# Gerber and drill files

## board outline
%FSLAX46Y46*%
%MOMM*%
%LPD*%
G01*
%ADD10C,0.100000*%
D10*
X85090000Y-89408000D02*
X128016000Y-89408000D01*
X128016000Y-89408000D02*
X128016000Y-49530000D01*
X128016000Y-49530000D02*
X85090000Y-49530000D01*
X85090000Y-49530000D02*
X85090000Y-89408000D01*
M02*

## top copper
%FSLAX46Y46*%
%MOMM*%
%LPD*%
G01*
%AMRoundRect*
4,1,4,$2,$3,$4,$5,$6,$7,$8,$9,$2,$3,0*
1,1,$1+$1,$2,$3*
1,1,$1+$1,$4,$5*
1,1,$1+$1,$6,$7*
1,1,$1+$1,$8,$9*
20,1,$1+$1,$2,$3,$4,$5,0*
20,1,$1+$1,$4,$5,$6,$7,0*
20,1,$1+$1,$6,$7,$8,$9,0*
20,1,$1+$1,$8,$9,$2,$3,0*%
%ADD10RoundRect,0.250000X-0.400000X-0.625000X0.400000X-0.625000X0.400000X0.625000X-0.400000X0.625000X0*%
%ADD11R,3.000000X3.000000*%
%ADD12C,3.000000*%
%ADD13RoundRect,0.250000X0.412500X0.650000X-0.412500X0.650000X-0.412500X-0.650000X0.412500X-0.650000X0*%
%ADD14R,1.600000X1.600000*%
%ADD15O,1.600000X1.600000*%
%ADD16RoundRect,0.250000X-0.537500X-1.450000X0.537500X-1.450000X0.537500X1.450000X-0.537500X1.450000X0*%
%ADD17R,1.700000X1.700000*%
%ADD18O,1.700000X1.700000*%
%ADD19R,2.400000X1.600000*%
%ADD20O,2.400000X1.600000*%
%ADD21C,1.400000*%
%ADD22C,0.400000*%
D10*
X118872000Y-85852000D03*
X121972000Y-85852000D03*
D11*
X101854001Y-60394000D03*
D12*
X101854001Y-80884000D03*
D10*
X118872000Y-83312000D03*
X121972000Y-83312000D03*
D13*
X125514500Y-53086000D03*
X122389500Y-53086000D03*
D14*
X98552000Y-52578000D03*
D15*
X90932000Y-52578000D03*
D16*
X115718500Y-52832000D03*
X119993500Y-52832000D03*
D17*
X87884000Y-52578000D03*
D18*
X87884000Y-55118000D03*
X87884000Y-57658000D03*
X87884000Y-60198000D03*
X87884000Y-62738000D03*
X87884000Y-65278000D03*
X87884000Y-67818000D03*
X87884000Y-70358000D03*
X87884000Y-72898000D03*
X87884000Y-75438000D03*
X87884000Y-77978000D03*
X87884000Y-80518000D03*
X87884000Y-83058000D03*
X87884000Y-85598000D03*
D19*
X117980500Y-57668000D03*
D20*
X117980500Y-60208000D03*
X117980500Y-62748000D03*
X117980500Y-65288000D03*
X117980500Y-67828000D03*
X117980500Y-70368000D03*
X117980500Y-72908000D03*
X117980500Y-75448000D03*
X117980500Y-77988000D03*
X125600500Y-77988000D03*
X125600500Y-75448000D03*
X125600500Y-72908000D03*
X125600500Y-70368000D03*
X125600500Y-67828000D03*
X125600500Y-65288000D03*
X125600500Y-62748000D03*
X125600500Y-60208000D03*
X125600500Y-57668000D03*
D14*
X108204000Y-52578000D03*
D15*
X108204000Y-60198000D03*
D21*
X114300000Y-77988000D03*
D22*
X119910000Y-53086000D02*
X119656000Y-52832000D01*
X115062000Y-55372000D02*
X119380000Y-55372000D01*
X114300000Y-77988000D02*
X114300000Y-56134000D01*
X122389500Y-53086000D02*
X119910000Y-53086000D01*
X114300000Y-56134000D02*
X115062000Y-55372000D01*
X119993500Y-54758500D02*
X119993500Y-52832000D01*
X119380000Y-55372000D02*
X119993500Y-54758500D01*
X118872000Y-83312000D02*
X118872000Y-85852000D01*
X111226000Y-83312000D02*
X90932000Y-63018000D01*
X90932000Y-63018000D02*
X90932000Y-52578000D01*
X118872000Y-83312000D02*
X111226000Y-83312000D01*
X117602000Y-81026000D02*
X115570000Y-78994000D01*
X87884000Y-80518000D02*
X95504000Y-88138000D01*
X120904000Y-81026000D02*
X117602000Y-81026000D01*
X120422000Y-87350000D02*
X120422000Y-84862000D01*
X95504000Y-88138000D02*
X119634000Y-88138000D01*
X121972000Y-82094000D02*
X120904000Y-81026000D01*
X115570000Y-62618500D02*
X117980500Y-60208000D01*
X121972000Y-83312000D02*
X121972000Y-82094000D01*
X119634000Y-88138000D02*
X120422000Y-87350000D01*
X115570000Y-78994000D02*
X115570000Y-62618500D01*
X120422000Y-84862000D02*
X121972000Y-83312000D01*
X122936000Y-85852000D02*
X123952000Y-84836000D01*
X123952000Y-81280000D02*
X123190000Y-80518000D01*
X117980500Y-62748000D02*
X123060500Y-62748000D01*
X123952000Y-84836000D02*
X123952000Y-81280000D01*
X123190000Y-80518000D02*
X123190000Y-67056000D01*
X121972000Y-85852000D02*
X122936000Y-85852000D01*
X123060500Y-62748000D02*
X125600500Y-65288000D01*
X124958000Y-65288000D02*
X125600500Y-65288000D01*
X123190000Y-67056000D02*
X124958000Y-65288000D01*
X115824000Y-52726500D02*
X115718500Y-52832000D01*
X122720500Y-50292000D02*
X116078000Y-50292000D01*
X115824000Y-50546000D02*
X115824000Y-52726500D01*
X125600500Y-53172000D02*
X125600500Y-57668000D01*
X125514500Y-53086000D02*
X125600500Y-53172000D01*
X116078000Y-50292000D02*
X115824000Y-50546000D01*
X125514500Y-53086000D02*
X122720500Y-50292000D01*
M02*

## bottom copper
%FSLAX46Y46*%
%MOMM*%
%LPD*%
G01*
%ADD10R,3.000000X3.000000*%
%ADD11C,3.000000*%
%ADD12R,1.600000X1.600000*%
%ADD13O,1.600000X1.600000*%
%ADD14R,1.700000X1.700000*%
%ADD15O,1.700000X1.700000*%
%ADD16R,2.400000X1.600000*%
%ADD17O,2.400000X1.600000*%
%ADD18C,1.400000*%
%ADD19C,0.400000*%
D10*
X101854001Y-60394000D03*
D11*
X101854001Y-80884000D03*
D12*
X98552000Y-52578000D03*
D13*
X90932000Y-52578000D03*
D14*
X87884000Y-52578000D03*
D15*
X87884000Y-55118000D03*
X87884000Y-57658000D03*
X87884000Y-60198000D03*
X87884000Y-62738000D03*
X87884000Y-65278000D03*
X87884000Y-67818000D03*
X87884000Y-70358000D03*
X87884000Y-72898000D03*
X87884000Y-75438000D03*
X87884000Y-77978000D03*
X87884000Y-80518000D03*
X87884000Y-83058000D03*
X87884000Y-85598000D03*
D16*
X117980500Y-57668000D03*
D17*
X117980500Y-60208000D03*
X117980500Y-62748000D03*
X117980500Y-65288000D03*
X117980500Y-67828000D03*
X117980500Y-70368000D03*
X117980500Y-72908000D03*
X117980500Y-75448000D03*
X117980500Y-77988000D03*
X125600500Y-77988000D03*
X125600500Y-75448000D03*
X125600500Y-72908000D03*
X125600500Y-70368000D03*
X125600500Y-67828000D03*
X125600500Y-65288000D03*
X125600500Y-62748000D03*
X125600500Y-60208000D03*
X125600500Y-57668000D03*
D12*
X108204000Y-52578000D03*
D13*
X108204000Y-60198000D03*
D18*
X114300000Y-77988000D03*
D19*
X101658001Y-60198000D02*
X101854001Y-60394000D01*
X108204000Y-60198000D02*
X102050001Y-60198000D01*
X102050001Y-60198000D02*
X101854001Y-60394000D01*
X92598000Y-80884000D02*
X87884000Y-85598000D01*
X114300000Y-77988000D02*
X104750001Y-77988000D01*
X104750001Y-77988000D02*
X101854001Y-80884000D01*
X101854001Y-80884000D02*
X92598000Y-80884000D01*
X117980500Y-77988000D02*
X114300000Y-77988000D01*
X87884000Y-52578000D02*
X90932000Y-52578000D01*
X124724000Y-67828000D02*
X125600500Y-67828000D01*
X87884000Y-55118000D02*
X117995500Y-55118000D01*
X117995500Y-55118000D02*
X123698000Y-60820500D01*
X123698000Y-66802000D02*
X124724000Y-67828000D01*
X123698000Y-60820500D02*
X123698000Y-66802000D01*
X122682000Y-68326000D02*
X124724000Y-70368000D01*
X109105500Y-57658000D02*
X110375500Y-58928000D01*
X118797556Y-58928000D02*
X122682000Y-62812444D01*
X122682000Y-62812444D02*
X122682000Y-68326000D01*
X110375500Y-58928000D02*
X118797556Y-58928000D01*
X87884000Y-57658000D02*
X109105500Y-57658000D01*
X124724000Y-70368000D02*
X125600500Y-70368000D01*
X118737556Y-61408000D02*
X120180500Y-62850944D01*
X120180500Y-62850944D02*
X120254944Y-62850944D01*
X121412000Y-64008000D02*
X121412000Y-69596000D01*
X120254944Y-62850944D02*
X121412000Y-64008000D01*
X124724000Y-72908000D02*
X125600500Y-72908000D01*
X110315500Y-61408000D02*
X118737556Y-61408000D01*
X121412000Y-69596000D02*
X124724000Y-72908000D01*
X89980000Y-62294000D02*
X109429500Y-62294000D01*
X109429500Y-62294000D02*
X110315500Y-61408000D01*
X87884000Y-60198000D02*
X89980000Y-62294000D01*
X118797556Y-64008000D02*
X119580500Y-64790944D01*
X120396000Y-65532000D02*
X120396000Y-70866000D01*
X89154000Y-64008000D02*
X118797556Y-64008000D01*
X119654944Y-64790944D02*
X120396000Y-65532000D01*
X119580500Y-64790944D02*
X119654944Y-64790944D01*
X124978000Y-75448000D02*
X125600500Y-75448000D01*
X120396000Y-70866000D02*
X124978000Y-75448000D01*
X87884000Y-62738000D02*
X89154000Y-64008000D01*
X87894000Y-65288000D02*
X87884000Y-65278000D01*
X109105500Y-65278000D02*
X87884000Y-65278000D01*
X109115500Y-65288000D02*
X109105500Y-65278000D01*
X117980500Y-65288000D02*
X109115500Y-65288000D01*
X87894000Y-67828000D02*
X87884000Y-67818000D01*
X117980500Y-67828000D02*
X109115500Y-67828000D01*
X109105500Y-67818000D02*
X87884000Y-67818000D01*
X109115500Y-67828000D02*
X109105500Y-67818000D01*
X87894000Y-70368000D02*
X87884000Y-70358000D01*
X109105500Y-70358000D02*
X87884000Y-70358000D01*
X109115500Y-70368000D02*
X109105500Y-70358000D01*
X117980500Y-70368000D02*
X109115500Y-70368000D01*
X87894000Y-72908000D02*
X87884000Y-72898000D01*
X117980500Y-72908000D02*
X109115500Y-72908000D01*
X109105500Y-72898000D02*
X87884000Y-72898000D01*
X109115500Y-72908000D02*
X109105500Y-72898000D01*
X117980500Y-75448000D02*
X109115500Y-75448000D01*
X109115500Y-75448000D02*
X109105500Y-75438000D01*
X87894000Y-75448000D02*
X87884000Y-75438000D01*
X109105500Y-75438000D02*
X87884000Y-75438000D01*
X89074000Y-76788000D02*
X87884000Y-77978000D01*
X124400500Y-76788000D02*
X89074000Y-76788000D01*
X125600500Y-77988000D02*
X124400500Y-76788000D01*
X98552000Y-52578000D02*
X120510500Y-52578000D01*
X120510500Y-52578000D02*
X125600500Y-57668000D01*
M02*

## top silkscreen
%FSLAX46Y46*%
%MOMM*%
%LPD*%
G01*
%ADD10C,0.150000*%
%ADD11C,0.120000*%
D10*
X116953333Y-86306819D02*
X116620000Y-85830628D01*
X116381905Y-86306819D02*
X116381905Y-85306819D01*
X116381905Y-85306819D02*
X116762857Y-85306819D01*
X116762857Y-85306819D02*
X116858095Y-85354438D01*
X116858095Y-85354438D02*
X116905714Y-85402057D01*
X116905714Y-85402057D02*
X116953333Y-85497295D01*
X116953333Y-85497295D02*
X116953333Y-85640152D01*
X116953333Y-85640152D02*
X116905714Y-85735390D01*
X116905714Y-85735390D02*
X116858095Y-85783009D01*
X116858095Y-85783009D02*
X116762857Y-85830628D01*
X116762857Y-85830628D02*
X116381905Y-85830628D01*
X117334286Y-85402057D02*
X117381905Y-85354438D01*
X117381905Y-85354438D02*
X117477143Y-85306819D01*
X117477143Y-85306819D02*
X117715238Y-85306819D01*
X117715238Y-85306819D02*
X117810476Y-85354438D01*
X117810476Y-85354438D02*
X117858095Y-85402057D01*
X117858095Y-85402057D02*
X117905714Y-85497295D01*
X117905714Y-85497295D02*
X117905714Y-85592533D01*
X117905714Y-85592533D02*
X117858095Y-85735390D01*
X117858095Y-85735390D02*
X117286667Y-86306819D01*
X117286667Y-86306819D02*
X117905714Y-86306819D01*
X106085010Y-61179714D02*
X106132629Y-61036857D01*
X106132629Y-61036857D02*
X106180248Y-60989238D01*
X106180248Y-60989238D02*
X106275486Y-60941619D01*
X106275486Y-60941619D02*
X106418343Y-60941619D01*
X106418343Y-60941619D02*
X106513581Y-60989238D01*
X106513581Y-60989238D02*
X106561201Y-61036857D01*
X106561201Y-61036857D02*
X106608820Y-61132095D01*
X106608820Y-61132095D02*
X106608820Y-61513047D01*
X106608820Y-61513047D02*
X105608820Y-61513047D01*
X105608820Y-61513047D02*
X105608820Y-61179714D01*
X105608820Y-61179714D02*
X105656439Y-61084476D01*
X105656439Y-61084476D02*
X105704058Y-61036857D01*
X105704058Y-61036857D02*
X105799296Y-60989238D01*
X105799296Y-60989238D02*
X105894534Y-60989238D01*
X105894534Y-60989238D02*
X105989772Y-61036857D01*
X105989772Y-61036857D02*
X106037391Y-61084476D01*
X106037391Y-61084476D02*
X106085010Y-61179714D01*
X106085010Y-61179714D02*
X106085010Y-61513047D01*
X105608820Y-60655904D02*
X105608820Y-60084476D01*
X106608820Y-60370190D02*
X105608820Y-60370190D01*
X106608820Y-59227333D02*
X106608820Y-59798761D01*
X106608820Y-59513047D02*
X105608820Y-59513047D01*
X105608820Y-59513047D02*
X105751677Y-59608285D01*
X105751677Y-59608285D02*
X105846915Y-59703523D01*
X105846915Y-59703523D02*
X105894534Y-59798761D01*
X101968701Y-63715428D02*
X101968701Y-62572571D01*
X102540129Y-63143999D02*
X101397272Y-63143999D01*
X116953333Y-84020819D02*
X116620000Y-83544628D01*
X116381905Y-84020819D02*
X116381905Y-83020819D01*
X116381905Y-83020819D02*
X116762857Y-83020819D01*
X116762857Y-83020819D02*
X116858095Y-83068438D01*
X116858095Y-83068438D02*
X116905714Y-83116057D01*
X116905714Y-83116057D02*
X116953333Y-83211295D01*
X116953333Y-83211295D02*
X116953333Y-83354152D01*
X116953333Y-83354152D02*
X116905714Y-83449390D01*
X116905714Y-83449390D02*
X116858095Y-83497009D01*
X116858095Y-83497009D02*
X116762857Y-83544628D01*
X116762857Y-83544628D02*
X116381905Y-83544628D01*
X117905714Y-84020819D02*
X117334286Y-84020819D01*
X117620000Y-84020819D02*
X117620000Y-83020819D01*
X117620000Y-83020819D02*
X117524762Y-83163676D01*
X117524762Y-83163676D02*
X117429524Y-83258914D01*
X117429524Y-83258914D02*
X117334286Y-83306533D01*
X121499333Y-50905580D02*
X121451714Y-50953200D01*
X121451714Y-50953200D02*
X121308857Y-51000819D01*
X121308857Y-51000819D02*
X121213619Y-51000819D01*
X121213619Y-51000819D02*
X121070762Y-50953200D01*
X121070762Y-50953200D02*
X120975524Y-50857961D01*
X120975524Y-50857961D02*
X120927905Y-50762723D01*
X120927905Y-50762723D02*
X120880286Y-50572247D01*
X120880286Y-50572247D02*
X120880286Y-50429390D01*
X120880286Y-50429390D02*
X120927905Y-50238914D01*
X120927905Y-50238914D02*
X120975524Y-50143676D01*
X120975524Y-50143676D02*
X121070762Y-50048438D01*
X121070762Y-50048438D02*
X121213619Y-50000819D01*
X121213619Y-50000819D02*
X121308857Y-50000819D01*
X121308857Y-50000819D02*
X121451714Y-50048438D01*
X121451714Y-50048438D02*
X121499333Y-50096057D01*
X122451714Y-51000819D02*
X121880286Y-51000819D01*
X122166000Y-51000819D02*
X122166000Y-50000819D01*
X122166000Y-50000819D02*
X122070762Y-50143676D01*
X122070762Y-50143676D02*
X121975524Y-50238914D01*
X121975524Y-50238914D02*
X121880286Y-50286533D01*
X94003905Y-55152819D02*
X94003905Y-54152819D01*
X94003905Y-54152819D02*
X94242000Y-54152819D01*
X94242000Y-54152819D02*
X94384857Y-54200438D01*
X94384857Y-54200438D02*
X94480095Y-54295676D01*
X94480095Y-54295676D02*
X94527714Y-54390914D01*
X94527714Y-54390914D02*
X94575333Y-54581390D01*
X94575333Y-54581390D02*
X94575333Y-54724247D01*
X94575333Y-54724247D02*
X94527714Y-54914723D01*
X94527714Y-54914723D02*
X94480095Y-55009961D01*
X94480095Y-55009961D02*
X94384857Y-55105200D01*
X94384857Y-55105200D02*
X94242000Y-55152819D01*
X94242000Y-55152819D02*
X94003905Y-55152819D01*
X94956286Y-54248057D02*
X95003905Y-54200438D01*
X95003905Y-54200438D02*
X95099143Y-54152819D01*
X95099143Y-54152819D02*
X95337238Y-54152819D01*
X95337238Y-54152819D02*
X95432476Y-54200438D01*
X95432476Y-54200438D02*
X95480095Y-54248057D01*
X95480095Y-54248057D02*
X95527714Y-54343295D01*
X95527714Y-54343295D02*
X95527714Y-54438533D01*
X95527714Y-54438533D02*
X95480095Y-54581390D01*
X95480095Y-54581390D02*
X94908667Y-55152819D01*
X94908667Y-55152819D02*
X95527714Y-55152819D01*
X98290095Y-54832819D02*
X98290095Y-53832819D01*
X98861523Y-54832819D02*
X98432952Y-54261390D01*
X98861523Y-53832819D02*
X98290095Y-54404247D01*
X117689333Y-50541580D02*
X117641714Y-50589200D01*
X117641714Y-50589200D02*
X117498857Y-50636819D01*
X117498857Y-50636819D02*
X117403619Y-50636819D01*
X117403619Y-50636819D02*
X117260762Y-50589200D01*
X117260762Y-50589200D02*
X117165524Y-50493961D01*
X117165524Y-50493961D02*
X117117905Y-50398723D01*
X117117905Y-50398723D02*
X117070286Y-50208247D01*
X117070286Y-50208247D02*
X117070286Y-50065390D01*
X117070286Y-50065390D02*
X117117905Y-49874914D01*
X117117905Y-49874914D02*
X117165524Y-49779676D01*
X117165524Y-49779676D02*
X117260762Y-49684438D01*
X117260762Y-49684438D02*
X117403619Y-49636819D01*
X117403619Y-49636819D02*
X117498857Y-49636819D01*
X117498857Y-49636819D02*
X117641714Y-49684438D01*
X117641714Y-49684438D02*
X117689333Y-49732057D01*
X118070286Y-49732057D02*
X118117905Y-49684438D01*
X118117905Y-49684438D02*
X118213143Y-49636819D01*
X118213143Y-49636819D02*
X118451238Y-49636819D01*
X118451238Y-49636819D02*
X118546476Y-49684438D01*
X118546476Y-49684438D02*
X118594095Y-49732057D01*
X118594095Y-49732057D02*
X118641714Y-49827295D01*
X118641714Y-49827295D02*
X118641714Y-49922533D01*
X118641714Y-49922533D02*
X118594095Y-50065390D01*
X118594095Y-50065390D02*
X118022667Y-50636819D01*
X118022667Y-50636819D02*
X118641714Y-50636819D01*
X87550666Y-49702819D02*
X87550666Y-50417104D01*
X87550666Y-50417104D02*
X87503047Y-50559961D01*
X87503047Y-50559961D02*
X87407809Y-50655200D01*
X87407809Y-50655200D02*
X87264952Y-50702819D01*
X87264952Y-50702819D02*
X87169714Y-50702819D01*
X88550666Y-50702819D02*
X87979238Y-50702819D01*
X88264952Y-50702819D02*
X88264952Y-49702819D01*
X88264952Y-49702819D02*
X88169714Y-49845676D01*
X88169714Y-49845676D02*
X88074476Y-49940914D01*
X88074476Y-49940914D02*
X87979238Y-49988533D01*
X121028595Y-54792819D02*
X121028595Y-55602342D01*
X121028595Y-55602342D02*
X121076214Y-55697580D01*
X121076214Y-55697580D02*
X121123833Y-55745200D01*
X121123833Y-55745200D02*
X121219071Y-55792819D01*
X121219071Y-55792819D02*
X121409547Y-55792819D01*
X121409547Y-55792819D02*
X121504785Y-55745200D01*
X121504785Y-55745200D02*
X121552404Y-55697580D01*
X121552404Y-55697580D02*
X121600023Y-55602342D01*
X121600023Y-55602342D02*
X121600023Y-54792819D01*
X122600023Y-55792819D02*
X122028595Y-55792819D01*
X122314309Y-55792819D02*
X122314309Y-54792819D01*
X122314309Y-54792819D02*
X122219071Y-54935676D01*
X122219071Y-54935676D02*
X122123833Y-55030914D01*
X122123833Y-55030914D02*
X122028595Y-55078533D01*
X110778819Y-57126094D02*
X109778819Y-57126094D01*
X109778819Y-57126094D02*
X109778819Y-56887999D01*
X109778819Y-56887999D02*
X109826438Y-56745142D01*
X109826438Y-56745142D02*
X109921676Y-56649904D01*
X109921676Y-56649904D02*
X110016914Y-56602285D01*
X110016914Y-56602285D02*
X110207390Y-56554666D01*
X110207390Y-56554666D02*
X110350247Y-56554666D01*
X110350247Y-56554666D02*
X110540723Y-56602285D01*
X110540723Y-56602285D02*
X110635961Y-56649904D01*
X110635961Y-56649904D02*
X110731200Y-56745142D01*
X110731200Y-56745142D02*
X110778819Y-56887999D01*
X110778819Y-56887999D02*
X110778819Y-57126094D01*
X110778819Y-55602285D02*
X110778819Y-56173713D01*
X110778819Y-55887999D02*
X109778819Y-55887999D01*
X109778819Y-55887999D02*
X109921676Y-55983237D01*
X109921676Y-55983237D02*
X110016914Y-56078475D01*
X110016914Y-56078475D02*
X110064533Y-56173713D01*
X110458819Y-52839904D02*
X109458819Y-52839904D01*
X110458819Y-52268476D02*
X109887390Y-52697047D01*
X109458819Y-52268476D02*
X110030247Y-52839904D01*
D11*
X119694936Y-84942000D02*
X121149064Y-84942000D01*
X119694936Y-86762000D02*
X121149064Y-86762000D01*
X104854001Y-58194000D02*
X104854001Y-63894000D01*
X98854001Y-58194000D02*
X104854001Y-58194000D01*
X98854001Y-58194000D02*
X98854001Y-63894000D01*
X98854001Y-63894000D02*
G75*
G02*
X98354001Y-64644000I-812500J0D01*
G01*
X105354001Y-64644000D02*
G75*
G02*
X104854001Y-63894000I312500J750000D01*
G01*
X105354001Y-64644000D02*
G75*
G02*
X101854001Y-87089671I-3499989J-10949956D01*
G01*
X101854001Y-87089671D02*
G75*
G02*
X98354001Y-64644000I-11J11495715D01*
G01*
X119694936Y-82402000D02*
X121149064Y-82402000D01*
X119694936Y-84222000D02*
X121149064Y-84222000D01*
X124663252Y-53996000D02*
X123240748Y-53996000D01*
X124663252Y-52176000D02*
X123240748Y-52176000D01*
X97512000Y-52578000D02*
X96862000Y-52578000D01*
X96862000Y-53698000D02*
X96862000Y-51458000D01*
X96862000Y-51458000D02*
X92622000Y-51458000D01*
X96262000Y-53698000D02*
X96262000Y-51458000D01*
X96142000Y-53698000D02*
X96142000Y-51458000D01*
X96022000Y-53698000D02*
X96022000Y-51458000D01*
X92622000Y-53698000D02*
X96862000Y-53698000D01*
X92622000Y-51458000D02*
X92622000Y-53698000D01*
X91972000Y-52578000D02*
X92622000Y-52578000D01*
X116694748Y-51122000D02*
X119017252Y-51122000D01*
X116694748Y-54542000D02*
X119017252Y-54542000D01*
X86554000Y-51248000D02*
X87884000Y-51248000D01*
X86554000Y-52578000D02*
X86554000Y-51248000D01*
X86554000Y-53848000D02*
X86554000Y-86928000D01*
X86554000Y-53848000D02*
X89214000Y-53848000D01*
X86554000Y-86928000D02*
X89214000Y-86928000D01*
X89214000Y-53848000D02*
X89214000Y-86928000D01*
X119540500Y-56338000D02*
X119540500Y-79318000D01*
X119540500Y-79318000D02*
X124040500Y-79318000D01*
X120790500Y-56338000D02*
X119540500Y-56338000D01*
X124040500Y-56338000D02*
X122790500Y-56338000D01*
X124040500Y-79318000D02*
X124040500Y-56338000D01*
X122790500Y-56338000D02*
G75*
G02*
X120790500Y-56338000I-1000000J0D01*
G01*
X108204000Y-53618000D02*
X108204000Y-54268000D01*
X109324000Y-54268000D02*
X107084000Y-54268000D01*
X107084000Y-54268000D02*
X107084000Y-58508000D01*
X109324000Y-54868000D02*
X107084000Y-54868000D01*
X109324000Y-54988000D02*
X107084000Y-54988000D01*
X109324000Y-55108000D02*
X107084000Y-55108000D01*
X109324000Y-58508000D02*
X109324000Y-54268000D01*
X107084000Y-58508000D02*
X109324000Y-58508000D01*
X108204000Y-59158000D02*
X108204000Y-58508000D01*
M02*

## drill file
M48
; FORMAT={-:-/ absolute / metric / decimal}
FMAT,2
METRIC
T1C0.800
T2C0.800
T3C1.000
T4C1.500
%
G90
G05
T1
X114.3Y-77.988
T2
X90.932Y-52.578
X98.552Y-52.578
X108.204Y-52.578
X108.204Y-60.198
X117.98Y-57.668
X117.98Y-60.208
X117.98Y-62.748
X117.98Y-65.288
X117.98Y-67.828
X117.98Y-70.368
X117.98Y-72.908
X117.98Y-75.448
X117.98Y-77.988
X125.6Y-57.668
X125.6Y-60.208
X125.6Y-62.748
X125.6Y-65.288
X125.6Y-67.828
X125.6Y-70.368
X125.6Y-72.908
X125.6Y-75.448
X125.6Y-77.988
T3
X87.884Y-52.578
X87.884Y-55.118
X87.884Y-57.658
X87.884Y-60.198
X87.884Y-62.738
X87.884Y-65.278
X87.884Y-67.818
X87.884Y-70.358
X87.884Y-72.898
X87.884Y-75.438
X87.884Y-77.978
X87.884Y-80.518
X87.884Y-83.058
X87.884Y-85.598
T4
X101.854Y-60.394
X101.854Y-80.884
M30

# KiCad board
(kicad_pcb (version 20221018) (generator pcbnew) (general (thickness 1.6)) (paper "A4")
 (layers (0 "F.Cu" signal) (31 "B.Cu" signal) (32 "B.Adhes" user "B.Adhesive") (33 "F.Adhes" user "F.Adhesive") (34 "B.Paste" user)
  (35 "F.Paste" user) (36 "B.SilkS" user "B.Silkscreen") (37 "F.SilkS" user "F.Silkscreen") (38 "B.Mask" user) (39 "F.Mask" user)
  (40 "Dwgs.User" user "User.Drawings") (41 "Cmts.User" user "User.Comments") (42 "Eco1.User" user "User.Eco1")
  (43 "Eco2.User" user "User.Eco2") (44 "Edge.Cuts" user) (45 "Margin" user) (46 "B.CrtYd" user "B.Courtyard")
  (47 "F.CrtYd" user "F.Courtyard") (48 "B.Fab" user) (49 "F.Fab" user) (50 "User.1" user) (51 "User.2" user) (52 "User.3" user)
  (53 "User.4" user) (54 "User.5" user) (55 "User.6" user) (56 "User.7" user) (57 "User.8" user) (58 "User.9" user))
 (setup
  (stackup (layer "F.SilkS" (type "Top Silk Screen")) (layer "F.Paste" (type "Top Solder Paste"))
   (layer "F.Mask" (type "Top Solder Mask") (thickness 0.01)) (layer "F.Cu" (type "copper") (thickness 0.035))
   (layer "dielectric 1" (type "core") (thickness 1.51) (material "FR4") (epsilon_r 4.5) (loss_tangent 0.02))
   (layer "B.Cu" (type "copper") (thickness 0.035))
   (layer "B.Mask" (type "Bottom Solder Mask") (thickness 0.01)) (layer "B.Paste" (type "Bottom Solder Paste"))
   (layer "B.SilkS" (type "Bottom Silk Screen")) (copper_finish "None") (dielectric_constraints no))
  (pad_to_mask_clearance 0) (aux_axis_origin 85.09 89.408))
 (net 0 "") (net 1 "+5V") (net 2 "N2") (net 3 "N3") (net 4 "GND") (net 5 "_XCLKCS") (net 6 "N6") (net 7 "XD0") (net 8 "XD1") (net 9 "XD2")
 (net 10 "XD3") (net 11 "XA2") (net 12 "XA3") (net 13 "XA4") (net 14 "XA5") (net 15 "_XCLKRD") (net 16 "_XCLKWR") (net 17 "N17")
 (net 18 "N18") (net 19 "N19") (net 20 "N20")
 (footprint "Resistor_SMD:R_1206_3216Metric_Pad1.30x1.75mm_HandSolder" (layer "F.Cu") (at 120.422 85.852)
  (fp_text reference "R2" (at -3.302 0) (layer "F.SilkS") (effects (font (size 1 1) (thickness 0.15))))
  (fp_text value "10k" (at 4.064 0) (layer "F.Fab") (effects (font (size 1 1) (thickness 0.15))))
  (fp_line (start -0.727064 -0.91) (end 0.727064 -0.91) (stroke (width 0.12) (type solid)) (layer "F.SilkS"))
  (fp_line (start -0.727064 0.91) (end 0.727064 0.91) (stroke (width 0.12) (type solid)) (layer "F.SilkS"))
  (pad "1" smd roundrect (at -1.55 0) (size 1.3 1.75) (layers "F.Cu" "F.Paste" "F.Mask") (roundrect_rratio 0.1923076923) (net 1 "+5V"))
  (pad "2" smd roundrect (at 1.55 0) (size 1.3 1.75) (layers "F.Cu" "F.Paste" "F.Mask") (roundrect_rratio 0.1923076923) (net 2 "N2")))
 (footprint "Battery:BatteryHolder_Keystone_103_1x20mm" (layer "F.Cu") (at 101.854001 60.394 -90)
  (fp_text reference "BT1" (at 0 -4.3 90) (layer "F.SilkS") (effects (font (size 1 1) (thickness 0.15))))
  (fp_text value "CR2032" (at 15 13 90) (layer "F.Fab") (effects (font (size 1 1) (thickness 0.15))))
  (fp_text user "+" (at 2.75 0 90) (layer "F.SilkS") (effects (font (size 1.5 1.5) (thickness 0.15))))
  (fp_line (start -2.2 -3) (end 3.5 -3) (stroke (width 0.12) (type solid)) (layer "F.SilkS"))
  (fp_line (start -2.2 3) (end -2.2 -3) (stroke (width 0.12) (type solid)) (layer "F.SilkS"))
  (fp_line (start -2.2 3) (end 3.5 3) (stroke (width 0.12) (type solid)) (layer "F.SilkS"))
  (fp_arc (start 3.5 3) (mid 3.950694 3.136459) (end 4.25 3.5) (stroke (width 0.12) (type solid)) (layer "F.SilkS"))
  (fp_arc (start 4.25 -3.5) (mid 3.950694 -3.136459) (end 3.5 -3) (stroke (width 0.12) (type solid)) (layer "F.SilkS"))
  (fp_arc (start 4.25 -3.5) (mid 16.971103 -11.358466) (end 26.695671 0) (stroke (width 0.12) (type solid)) (layer "F.SilkS"))
  (fp_arc (start 26.695671 0) (mid 16.971103 11.358466) (end 4.25 3.5) (stroke (width 0.12) (type solid)) (layer "F.SilkS"))
  (pad "1" thru_hole rect (at 0 0 270) (size 3 3) (drill 1.5) (layers "*.Cu" "*.Mask") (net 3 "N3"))
  (pad "2" thru_hole circle (at 20.49 0 270) (size 3 3) (drill 1.5) (layers "*.Cu" "*.Mask") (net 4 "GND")))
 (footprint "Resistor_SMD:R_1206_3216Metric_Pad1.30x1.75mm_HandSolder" (layer "F.Cu") (at 120.422 83.312)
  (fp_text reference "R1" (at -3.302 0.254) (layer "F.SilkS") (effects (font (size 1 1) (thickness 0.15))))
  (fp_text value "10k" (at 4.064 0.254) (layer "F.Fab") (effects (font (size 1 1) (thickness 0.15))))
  (fp_line (start -0.727064 -0.91) (end 0.727064 -0.91) (stroke (width 0.12) (type solid)) (layer "F.SilkS"))
  (fp_line (start -0.727064 0.91) (end 0.727064 0.91) (stroke (width 0.12) (type solid)) (layer "F.SilkS"))
  (pad "1" smd roundrect (at -1.55 0) (size 1.3 1.75) (layers "F.Cu" "F.Paste" "F.Mask") (roundrect_rratio 0.1923076923) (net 1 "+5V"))
  (pad "2" smd roundrect (at 1.55 0) (size 1.3 1.75) (layers "F.Cu" "F.Paste" "F.Mask") (roundrect_rratio 0.1923076923) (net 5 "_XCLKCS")))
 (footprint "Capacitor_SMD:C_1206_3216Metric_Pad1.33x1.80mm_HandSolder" (layer "F.Cu") (at 123.952 53.086 180)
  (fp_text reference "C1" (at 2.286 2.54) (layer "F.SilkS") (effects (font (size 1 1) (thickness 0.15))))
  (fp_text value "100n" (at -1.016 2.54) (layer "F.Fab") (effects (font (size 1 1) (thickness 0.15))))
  (fp_line (start -0.711252 -0.91) (end 0.711252 -0.91) (stroke (width 0.12) (type solid)) (layer "F.SilkS"))
  (fp_line (start -0.711252 0.91) (end 0.711252 0.91) (stroke (width 0.12) (type solid)) (layer "F.SilkS"))
  (pad "1" smd roundrect (at -1.5625 0 180) (size 1.325 1.8) (layers "F.Cu" "F.Paste" "F.Mask") (roundrect_rratio 0.1886792453) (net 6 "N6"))
  (pad "2" smd roundrect (at 1.5625 0 180) (size 1.325 1.8) (layers "F.Cu" "F.Paste" "F.Mask") (roundrect_rratio 0.1886792453) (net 4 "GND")))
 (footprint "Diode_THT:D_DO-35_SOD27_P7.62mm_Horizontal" (layer "F.Cu") (at 98.552 52.578 180)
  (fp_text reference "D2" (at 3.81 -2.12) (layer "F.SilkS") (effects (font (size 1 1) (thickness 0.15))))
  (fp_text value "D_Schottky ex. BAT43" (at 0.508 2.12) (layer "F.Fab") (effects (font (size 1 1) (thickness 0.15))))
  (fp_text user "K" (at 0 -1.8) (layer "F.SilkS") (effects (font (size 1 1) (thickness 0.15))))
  (fp_line (start 1.04 0) (end 1.69 0) (stroke (width 0.12) (type solid)) (layer "F.SilkS"))
  (fp_line (start 1.69 -1.12) (end 1.69 1.12) (stroke (width 0.12) (type solid)) (layer "F.SilkS"))
  (fp_line (start 1.69 1.12) (end 5.93 1.12) (stroke (width 0.12) (type solid)) (layer "F.SilkS"))
  (fp_line (start 2.29 -1.12) (end 2.29 1.12) (stroke (width 0.12) (type solid)) (layer "F.SilkS"))
  (fp_line (start 2.41 -1.12) (end 2.41 1.12) (stroke (width 0.12) (type solid)) (layer "F.SilkS"))
  (fp_line (start 2.53 -1.12) (end 2.53 1.12) (stroke (width 0.12) (type solid)) (layer "F.SilkS"))
  (fp_line (start 5.93 -1.12) (end 1.69 -1.12) (stroke (width 0.12) (type solid)) (layer "F.SilkS"))
  (fp_line (start 5.93 1.12) (end 5.93 -1.12) (stroke (width 0.12) (type solid)) (layer "F.SilkS"))
  (fp_line (start 6.58 0) (end 5.93 0) (stroke (width 0.12) (type solid)) (layer "F.SilkS"))
  (pad "1" thru_hole rect (at 0 0 180) (size 1.6 1.6) (drill 0.8) (layers "*.Cu" "*.Mask") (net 6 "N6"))
  (pad "2" thru_hole oval (at 7.62 0 180) (size 1.6 1.6) (drill 0.8) (layers "*.Cu" "*.Mask") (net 1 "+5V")))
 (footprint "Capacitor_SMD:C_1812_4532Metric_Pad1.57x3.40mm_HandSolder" (layer "F.Cu") (at 117.856 52.832)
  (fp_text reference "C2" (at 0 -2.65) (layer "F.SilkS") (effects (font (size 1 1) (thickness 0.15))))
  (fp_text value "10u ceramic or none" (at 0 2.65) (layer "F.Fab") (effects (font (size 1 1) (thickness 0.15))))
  (fp_line (start -1.161252 -1.71) (end 1.161252 -1.71) (stroke (width 0.12) (type solid)) (layer "F.SilkS"))
  (fp_line (start -1.161252 1.71) (end 1.161252 1.71) (stroke (width 0.12) (type solid)) (layer "F.SilkS"))
  (pad "1" smd roundrect (at -2.1375 0) (size 1.575 3.4) (layers "F.Cu" "F.Paste" "F.Mask") (roundrect_rratio 0.15873) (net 6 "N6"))
  (pad "2" smd roundrect (at 2.1375 0) (size 1.575 3.4) (layers "F.Cu" "F.Paste" "F.Mask") (roundrect_rratio 0.15873) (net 4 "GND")))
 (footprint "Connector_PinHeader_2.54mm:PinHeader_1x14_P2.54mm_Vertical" (layer "F.Cu") (at 87.884 52.578)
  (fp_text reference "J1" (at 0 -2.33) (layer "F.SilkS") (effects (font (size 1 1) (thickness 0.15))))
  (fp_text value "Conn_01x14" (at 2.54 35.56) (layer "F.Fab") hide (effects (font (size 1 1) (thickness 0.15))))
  (fp_line (start -1.33 -1.33) (end 0 -1.33) (stroke (width 0.12) (type solid)) (layer "F.SilkS"))
  (fp_line (start -1.33 0) (end -1.33 -1.33) (stroke (width 0.12) (type solid)) (layer "F.SilkS"))
  (fp_line (start -1.33 1.27) (end -1.33 34.35) (stroke (width 0.12) (type solid)) (layer "F.SilkS"))
  (fp_line (start -1.33 1.27) (end 1.33 1.27) (stroke (width 0.12) (type solid)) (layer "F.SilkS"))
  (fp_line (start -1.33 34.35) (end 1.33 34.35) (stroke (width 0.12) (type solid)) (layer "F.SilkS"))
  (fp_line (start 1.33 1.27) (end 1.33 34.35) (stroke (width 0.12) (type solid)) (layer "F.SilkS"))
  (pad "1" thru_hole rect (at 0 0) (size 1.7 1.7) (drill 1) (layers "*.Cu" "*.Mask") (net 1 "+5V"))
  (pad "2" thru_hole oval (at 0 2.54) (size 1.7 1.7) (drill 1) (layers "*.Cu" "*.Mask") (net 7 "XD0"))
  (pad "3" thru_hole oval (at 0 5.08) (size 1.7 1.7) (drill 1) (layers "*.Cu" "*.Mask") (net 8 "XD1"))
  (pad "4" thru_hole oval (at 0 7.62) (size 1.7 1.7) (drill 1) (layers "*.Cu" "*.Mask") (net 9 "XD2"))
  (pad "5" thru_hole oval (at 0 10.16) (size 1.7 1.7) (drill 1) (layers "*.Cu" "*.Mask") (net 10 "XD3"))
  (pad "6" thru_hole oval (at 0 12.7) (size 1.7 1.7) (drill 1) (layers "*.Cu" "*.Mask") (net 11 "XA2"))
  (pad "7" thru_hole oval (at 0 15.24) (size 1.7 1.7) (drill 1) (layers "*.Cu" "*.Mask") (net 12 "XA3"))
  (pad "8" thru_hole oval (at 0 17.78) (size 1.7 1.7) (drill 1) (layers "*.Cu" "*.Mask") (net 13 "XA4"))
  (pad "9" thru_hole oval (at 0 20.32) (size 1.7 1.7) (drill 1) (layers "*.Cu" "*.Mask") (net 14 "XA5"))
  (pad "10" thru_hole oval (at 0 22.86) (size 1.7 1.7) (drill 1) (layers "*.Cu" "*.Mask") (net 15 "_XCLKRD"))
  (pad "11" thru_hole oval (at 0 25.4) (size 1.7 1.7) (drill 1) (layers "*.Cu" "*.Mask") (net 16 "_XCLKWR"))
  (pad "12" thru_hole oval (at 0 27.94) (size 1.7 1.7) (drill 1) (layers "*.Cu" "*.Mask") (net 5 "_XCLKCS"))
  (pad "13" thru_hole oval (at 0 30.48) (size 1.7 1.7) (drill 1) (layers "*.Cu" "*.Mask") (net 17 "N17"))
  (pad "14" thru_hole oval (at 0 33.02) (size 1.7 1.7) (drill 1) (layers "*.Cu" "*.Mask") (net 4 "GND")))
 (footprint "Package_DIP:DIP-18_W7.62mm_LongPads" (layer "F.Cu") (at 117.9805 57.668)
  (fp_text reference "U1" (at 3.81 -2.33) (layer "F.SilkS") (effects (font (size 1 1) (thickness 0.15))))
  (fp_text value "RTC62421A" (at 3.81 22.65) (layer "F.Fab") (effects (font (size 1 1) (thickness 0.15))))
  (fp_line (start 1.56 -1.33) (end 1.56 21.65) (stroke (width 0.12) (type solid)) (layer "F.SilkS"))
  (fp_line (start 1.56 21.65) (end 6.06 21.65) (stroke (width 0.12) (type solid)) (layer "F.SilkS"))
  (fp_line (start 2.81 -1.33) (end 1.56 -1.33) (stroke (width 0.12) (type solid)) (layer "F.SilkS"))
  (fp_line (start 6.06 -1.33) (end 4.81 -1.33) (stroke (width 0.12) (type solid)) (layer "F.SilkS"))
  (fp_line (start 6.06 21.65) (end 6.06 -1.33) (stroke (width 0.12) (type solid)) (layer "F.SilkS"))
  (fp_arc (start 4.81 -1.33) (mid 3.81 -0.33) (end 2.81 -1.33) (stroke (width 0.12) (type solid)) (layer "F.SilkS"))
  (pad "1" thru_hole rect (at 0 0) (size 2.4 1.6) (drill 0.8) (layers "*.Cu" "*.Mask") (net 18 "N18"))
  (pad "2" thru_hole oval (at 0 2.54) (size 2.4 1.6) (drill 0.8) (layers "*.Cu" "*.Mask") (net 5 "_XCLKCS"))
  (pad "3" thru_hole oval (at 0 5.08) (size 2.4 1.6) (drill 0.8) (layers "*.Cu" "*.Mask") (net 2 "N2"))
  (pad "4" thru_hole oval (at 0 7.62) (size 2.4 1.6) (drill 0.8) (layers "*.Cu" "*.Mask") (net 11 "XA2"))
  (pad "5" thru_hole oval (at 0 10.16) (size 2.4 1.6) (drill 0.8) (layers "*.Cu" "*.Mask") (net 12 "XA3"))
  (pad "6" thru_hole oval (at 0 12.7) (size 2.4 1.6) (drill 0.8) (layers "*.Cu" "*.Mask") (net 13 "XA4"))
  (pad "7" thru_hole oval (at 0 15.24) (size 2.4 1.6) (drill 0.8) (layers "*.Cu" "*.Mask") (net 14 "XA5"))
  (pad "8" thru_hole oval (at 0 17.78) (size 2.4 1.6) (drill 0.8) (layers "*.Cu" "*.Mask") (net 15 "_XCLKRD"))
  (pad "9" thru_hole oval (at 0 20.32) (size 2.4 1.6) (drill 0.8) (layers "*.Cu" "*.Mask") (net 4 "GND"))
  (pad "10" thru_hole oval (at 7.62 20.32) (size 2.4 1.6) (drill 0.8) (layers "*.Cu" "*.Mask") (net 16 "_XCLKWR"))
  (pad "11" thru_hole oval (at 7.62 17.78) (size 2.4 1.6) (drill 0.8) (layers "*.Cu" "*.Mask") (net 10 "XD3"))
  (pad "12" thru_hole oval (at 7.62 15.24) (size 2.4 1.6) (drill 0.8) (layers "*.Cu" "*.Mask") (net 9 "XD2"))
  (pad "13" thru_hole oval (at 7.62 12.7) (size 2.4 1.6) (drill 0.8) (layers "*.Cu" "*.Mask") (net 8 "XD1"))
  (pad "14" thru_hole oval (at 7.62 10.16) (size 2.4 1.6) (drill 0.8) (layers "*.Cu" "*.Mask") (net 7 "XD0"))
  (pad "15" thru_hole oval (at 7.62 7.62) (size 2.4 1.6) (drill 0.8) (layers "*.Cu" "*.Mask") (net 2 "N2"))
  (pad "16" thru_hole oval (at 7.62 5.08) (size 2.4 1.6) (drill 0.8) (layers "*.Cu" "*.Mask") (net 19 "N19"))
  (pad "17" thru_hole oval (at 7.62 2.54) (size 2.4 1.6) (drill 0.8) (layers "*.Cu" "*.Mask") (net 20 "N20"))
  (pad "18" thru_hole oval (at 7.62 0) (size 2.4 1.6) (drill 0.8) (layers "*.Cu" "*.Mask") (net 6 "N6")))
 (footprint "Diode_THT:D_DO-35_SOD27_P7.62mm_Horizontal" (layer "F.Cu") (at 108.204 52.578 -90)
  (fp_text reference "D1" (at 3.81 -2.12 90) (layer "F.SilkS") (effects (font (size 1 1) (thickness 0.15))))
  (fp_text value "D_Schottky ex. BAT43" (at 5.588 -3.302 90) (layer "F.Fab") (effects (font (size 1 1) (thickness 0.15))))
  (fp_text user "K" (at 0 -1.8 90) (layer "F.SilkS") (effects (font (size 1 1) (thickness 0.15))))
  (fp_line (start 1.04 0) (end 1.69 0) (stroke (width 0.12) (type solid)) (layer "F.SilkS"))
  (fp_line (start 1.69 -1.12) (end 1.69 1.12) (stroke (width 0.12) (type solid)) (layer "F.SilkS"))
  (fp_line (start 1.69 1.12) (end 5.93 1.12) (stroke (width 0.12) (type solid)) (layer "F.SilkS"))
  (fp_line (start 2.29 -1.12) (end 2.29 1.12) (stroke (width 0.12) (type solid)) (layer "F.SilkS"))
  (fp_line (start 2.41 -1.12) (end 2.41 1.12) (stroke (width 0.12) (type solid)) (layer "F.SilkS"))
  (fp_line (start 2.53 -1.12) (end 2.53 1.12) (stroke (width 0.12) (type solid)) (layer "F.SilkS"))
  (fp_line (start 5.93 -1.12) (end 1.69 -1.12) (stroke (width 0.12) (type solid)) (layer "F.SilkS"))
  (fp_line (start 5.93 1.12) (end 5.93 -1.12) (stroke (width 0.12) (type solid)) (layer "F.SilkS"))
  (fp_line (start 6.58 0) (end 5.93 0) (stroke (width 0.12) (type solid)) (layer "F.SilkS"))
  (pad "1" thru_hole rect (at 0 0 270) (size 1.6 1.6) (drill 0.8) (layers "*.Cu" "*.Mask") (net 6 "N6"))
  (pad "2" thru_hole oval (at 7.62 0 270) (size 1.6 1.6) (drill 0.8) (layers "*.Cu" "*.Mask") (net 3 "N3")))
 (gr_line (start 85.09 89.408) (end 128.016 89.408) (stroke (width 0.1) (type default)) (layer "Edge.Cuts"))
 (gr_line (start 128.016 89.408) (end 128.016 49.53) (stroke (width 0.1) (type default)) (layer "Edge.Cuts"))
 (gr_line (start 128.016 49.53) (end 85.09 49.53) (stroke (width 0.1) (type default)) (layer "Edge.Cuts"))
 (gr_line (start 85.09 49.53) (end 85.09 89.408) (stroke (width 0.1) (type default)) (layer "Edge.Cuts"))
 (segment (start 101.658001 60.198) (end 101.854001 60.394) (width 0.4) (layer "B.Cu") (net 3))
 (segment (start 108.204 60.198) (end 102.050001 60.198) (width 0.4) (layer "B.Cu") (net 3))
 (segment (start 102.050001 60.198) (end 101.854001 60.394) (width 0.4) (layer "B.Cu") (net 3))
 (segment (start 119.91 53.086) (end 119.656 52.832) (width 0.4) (layer "F.Cu") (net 4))
 (segment (start 115.062 55.372) (end 119.38 55.372) (width 0.4) (layer "F.Cu") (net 4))
 (segment (start 114.3 77.988) (end 114.3 56.134) (width 0.4) (layer "F.Cu") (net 4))
 (segment (start 122.3895 53.086) (end 119.91 53.086) (width 0.4) (layer "F.Cu") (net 4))
 (segment (start 114.3 56.134) (end 115.062 55.372) (width 0.4) (layer "F.Cu") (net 4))
 (segment (start 119.9935 54.7585) (end 119.9935 52.832) (width 0.4) (layer "F.Cu") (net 4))
 (segment (start 119.38 55.372) (end 119.9935 54.7585) (width 0.4) (layer "F.Cu") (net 4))
 (via (at 114.3 77.988) (size 1.4) (drill 0.8) (layers "F.Cu" "B.Cu") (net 4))
 (segment (start 92.598 80.884) (end 87.884 85.598) (width 0.4) (layer "B.Cu") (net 4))
 (segment (start 114.3 77.988) (end 104.750001 77.988) (width 0.4) (layer "B.Cu") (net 4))
 (segment (start 104.750001 77.988) (end 101.854001 80.884) (width 0.4) (layer "B.Cu") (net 4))
 (segment (start 101.854001 80.884) (end 92.598 80.884) (width 0.4) (layer "B.Cu") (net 4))
 (segment (start 117.9805 77.988) (end 114.3 77.988) (width 0.4) (layer "B.Cu") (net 4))
 (segment (start 118.872 83.312) (end 118.872 85.852) (width 0.4) (layer "F.Cu") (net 1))
 (segment (start 111.226 83.312) (end 90.932 63.018) (width 0.4) (layer "F.Cu") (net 1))
 (segment (start 90.932 63.018) (end 90.932 52.578) (width 0.4) (layer "F.Cu") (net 1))
 (segment (start 118.872 83.312) (end 111.226 83.312) (width 0.4) (layer "F.Cu") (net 1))
 (segment (start 87.884 52.578) (end 90.932 52.578) (width 0.4) (layer "B.Cu") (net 1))
 (segment (start 124.724 67.828) (end 125.6005 67.828) (width 0.4) (layer "B.Cu") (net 7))
 (segment (start 87.884 55.118) (end 117.9955 55.118) (width 0.4) (layer "B.Cu") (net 7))
 (segment (start 117.9955 55.118) (end 123.698 60.8205) (width 0.4) (layer "B.Cu") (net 7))
 (segment (start 123.698 66.802) (end 124.724 67.828) (width 0.4) (layer "B.Cu") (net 7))
 (segment (start 123.698 60.8205) (end 123.698 66.802) (width 0.4) (layer "B.Cu") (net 7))
 (segment (start 122.682 68.326) (end 124.724 70.368) (width 0.4) (layer "B.Cu") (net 8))
 (segment (start 109.1055 57.658) (end 110.3755 58.928) (width 0.4) (layer "B.Cu") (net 8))
 (segment (start 118.797556 58.928) (end 122.682 62.812444) (width 0.4) (layer "B.Cu") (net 8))
 (segment (start 122.682 62.812444) (end 122.682 68.326) (width 0.4) (layer "B.Cu") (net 8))
 (segment (start 110.3755 58.928) (end 118.797556 58.928) (width 0.4) (layer "B.Cu") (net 8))
 (segment (start 87.884 57.658) (end 109.1055 57.658) (width 0.4) (layer "B.Cu") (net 8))
 (segment (start 124.724 70.368) (end 125.6005 70.368) (width 0.4) (layer "B.Cu") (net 8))
 (segment (start 118.737556 61.408) (end 120.1805 62.850944) (width 0.4) (layer "B.Cu") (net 9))
 (segment (start 120.1805 62.850944) (end 120.254944 62.850944) (width 0.4) (layer "B.Cu") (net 9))
 (segment (start 121.412 64.008) (end 121.412 69.596) (width 0.4) (layer "B.Cu") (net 9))
 (segment (start 120.254944 62.850944) (end 121.412 64.008) (width 0.4) (layer "B.Cu") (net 9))
 (segment (start 124.724 72.908) (end 125.6005 72.908) (width 0.4) (layer "B.Cu") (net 9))
 (segment (start 110.3155 61.408) (end 118.737556 61.408) (width 0.4) (layer "B.Cu") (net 9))
 (segment (start 121.412 69.596) (end 124.724 72.908) (width 0.4) (layer "B.Cu") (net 9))
 (segment (start 89.98 62.294) (end 109.4295 62.294) (width 0.4) (layer "B.Cu") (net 9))
 (segment (start 109.4295 62.294) (end 110.3155 61.408) (width 0.4) (layer "B.Cu") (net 9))
 (segment (start 87.884 60.198) (end 89.98 62.294) (width 0.4) (layer "B.Cu") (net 9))
 (segment (start 118.797556 64.008) (end 119.5805 64.790944) (width 0.4) (layer "B.Cu") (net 10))
 (segment (start 120.396 65.532) (end 120.396 70.866) (width 0.4) (layer "B.Cu") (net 10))
 (segment (start 89.154 64.008) (end 118.797556 64.008) (width 0.4) (layer "B.Cu") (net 10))
 (segment (start 119.654944 64.790944) (end 120.396 65.532) (width 0.4) (layer "B.Cu") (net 10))
 (segment (start 119.5805 64.790944) (end 119.654944 64.790944) (width 0.4) (layer "B.Cu") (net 10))
 (segment (start 124.978 75.448) (end 125.6005 75.448) (width 0.4) (layer "B.Cu") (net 10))
 (segment (start 120.396 70.866) (end 124.978 75.448) (width 0.4) (layer "B.Cu") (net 10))
 (segment (start 87.884 62.738) (end 89.154 64.008) (width 0.4) (layer "B.Cu") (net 10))
 (segment (start 87.894 65.288) (end 87.884 65.278) (width 0.4) (layer "B.Cu") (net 11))
 (segment (start 109.1055 65.278) (end 87.884 65.278) (width 0.4) (layer "B.Cu") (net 11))
 (segment (start 109.1155 65.288) (end 109.1055 65.278) (width 0.4) (layer "B.Cu") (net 11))
 (segment (start 117.9805 65.288) (end 109.1155 65.288) (width 0.4) (layer "B.Cu") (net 11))
 (segment (start 87.894 67.828) (end 87.884 67.818) (width 0.4) (layer "B.Cu") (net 12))
 (segment (start 117.9805 67.828) (end 109.1155 67.828) (width 0.4) (layer "B.Cu") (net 12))
 (segment (start 109.1055 67.818) (end 87.884 67.818) (width 0.4) (layer "B.Cu") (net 12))
 (segment (start 109.1155 67.828) (end 109.1055 67.818) (width 0.4) (layer "B.Cu") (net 12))
 (segment (start 87.894 70.368) (end 87.884 70.358) (width 0.4) (layer "B.Cu") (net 13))
 (segment (start 109.1055 70.358) (end 87.884 70.358) (width 0.4) (layer "B.Cu") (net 13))
 (segment (start 109.1155 70.368) (end 109.1055 70.358) (width 0.4) (layer "B.Cu") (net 13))
 (segment (start 117.9805 70.368) (end 109.1155 70.368) (width 0.4) (layer "B.Cu") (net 13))
 (segment (start 87.894 72.908) (end 87.884 72.898) (width 0.4) (layer "B.Cu") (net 14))
 (segment (start 117.9805 72.908) (end 109.1155 72.908) (width 0.4) (layer "B.Cu") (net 14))
 (segment (start 109.1055 72.898) (end 87.884 72.898) (width 0.4) (layer "B.Cu") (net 14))
 (segment (start 109.1155 72.908) (end 109.1055 72.898) (width 0.4) (layer "B.Cu") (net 14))
 (segment (start 117.9805 75.448) (end 109.1155 75.448) (width 0.4) (layer "B.Cu") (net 15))
 (segment (start 109.1155 75.448) (end 109.1055 75.438) (width 0.4) (layer "B.Cu") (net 15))
 (segment (start 87.894 75.448) (end 87.884 75.438) (width 0.4) (layer "B.Cu") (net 15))
 (segment (start 109.1055 75.438) (end 87.884 75.438) (width 0.4) (layer "B.Cu") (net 15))
 (segment (start 89.074 76.788) (end 87.884 77.978) (width 0.4) (layer "B.Cu") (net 16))
 (segment (start 124.4005 76.788) (end 89.074 76.788) (width 0.4) (layer "B.Cu") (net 16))
 (segment (start 125.6005 77.988) (end 124.4005 76.788) (width 0.4) (layer "B.Cu") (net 16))
 (segment (start 117.602 81.026) (end 115.57 78.994) (width 0.4) (layer "F.Cu") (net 5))
 (segment (start 87.884 80.518) (end 95.504 88.138) (width 0.4) (layer "F.Cu") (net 5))
 (segment (start 120.904 81.026) (end 117.602 81.026) (width 0.4) (layer "F.Cu") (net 5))
 (segment (start 120.422 87.35) (end 120.422 84.862) (width 0.4) (layer "F.Cu") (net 5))
 (segment (start 95.504 88.138) (end 119.634 88.138) (width 0.4) (layer "F.Cu") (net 5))
 (segment (start 121.972 82.094) (end 120.904 81.026) (width 0.4) (layer "F.Cu") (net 5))
 (segment (start 115.57 62.6185) (end 117.9805 60.208) (width 0.4) (layer "F.Cu") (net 5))
 (segment (start 121.972 83.312) (end 121.972 82.094) (width 0.4) (layer "F.Cu") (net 5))
 (segment (start 119.634 88.138) (end 120.422 87.35) (width 0.4) (layer "F.Cu") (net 5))
 (segment (start 115.57 78.994) (end 115.57 62.6185) (width 0.4) (layer "F.Cu") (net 5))
 (segment (start 120.422 84.862) (end 121.972 83.312) (width 0.4) (layer "F.Cu") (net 5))
 (segment (start 122.936 85.852) (end 123.952 84.836) (width 0.4) (layer "F.Cu") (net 2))
 (segment (start 123.952 81.28) (end 123.19 80.518) (width 0.4) (layer "F.Cu") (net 2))
 (segment (start 117.9805 62.748) (end 123.0605 62.748) (width 0.4) (layer "F.Cu") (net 2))
 (segment (start 123.952 84.836) (end 123.952 81.28) (width 0.4) (layer "F.Cu") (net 2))
 (segment (start 123.19 80.518) (end 123.19 67.056) (width 0.4) (layer "F.Cu") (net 2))
 (segment (start 121.972 85.852) (end 122.936 85.852) (width 0.4) (layer "F.Cu") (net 2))
 (segment (start 123.0605 62.748) (end 125.6005 65.288) (width 0.4) (layer "F.Cu") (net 2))
 (segment (start 124.958 65.288) (end 125.6005 65.288) (width 0.4) (layer "F.Cu") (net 2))
 (segment (start 123.19 67.056) (end 124.958 65.288) (width 0.4) (layer "F.Cu") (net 2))
 (segment (start 115.824 52.7265) (end 115.7185 52.832) (width 0.4) (layer "F.Cu") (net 6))
 (segment (start 122.7205 50.292) (end 116.078 50.292) (width 0.4) (layer "F.Cu") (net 6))
 (segment (start 115.824 50.546) (end 115.824 52.7265) (width 0.4) (layer "F.Cu") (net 6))
 (segment (start 125.6005 53.172) (end 125.6005 57.668) (width 0.4) (layer "F.Cu") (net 6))
 (segment (start 125.5145 53.086) (end 125.6005 53.172) (width 0.4) (layer "F.Cu") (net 6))
 (segment (start 116.078 50.292) (end 115.824 50.546) (width 0.4) (layer "F.Cu") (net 6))
 (segment (start 125.5145 53.086) (end 122.7205 50.292) (width 0.4) (layer "F.Cu") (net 6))
 (segment (start 98.552 52.578) (end 120.5105 52.578) (width 0.4) (layer "B.Cu") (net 6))
 (segment (start 120.5105 52.578) (end 125.6005 57.668) (width 0.4) (layer "B.Cu") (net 6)))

